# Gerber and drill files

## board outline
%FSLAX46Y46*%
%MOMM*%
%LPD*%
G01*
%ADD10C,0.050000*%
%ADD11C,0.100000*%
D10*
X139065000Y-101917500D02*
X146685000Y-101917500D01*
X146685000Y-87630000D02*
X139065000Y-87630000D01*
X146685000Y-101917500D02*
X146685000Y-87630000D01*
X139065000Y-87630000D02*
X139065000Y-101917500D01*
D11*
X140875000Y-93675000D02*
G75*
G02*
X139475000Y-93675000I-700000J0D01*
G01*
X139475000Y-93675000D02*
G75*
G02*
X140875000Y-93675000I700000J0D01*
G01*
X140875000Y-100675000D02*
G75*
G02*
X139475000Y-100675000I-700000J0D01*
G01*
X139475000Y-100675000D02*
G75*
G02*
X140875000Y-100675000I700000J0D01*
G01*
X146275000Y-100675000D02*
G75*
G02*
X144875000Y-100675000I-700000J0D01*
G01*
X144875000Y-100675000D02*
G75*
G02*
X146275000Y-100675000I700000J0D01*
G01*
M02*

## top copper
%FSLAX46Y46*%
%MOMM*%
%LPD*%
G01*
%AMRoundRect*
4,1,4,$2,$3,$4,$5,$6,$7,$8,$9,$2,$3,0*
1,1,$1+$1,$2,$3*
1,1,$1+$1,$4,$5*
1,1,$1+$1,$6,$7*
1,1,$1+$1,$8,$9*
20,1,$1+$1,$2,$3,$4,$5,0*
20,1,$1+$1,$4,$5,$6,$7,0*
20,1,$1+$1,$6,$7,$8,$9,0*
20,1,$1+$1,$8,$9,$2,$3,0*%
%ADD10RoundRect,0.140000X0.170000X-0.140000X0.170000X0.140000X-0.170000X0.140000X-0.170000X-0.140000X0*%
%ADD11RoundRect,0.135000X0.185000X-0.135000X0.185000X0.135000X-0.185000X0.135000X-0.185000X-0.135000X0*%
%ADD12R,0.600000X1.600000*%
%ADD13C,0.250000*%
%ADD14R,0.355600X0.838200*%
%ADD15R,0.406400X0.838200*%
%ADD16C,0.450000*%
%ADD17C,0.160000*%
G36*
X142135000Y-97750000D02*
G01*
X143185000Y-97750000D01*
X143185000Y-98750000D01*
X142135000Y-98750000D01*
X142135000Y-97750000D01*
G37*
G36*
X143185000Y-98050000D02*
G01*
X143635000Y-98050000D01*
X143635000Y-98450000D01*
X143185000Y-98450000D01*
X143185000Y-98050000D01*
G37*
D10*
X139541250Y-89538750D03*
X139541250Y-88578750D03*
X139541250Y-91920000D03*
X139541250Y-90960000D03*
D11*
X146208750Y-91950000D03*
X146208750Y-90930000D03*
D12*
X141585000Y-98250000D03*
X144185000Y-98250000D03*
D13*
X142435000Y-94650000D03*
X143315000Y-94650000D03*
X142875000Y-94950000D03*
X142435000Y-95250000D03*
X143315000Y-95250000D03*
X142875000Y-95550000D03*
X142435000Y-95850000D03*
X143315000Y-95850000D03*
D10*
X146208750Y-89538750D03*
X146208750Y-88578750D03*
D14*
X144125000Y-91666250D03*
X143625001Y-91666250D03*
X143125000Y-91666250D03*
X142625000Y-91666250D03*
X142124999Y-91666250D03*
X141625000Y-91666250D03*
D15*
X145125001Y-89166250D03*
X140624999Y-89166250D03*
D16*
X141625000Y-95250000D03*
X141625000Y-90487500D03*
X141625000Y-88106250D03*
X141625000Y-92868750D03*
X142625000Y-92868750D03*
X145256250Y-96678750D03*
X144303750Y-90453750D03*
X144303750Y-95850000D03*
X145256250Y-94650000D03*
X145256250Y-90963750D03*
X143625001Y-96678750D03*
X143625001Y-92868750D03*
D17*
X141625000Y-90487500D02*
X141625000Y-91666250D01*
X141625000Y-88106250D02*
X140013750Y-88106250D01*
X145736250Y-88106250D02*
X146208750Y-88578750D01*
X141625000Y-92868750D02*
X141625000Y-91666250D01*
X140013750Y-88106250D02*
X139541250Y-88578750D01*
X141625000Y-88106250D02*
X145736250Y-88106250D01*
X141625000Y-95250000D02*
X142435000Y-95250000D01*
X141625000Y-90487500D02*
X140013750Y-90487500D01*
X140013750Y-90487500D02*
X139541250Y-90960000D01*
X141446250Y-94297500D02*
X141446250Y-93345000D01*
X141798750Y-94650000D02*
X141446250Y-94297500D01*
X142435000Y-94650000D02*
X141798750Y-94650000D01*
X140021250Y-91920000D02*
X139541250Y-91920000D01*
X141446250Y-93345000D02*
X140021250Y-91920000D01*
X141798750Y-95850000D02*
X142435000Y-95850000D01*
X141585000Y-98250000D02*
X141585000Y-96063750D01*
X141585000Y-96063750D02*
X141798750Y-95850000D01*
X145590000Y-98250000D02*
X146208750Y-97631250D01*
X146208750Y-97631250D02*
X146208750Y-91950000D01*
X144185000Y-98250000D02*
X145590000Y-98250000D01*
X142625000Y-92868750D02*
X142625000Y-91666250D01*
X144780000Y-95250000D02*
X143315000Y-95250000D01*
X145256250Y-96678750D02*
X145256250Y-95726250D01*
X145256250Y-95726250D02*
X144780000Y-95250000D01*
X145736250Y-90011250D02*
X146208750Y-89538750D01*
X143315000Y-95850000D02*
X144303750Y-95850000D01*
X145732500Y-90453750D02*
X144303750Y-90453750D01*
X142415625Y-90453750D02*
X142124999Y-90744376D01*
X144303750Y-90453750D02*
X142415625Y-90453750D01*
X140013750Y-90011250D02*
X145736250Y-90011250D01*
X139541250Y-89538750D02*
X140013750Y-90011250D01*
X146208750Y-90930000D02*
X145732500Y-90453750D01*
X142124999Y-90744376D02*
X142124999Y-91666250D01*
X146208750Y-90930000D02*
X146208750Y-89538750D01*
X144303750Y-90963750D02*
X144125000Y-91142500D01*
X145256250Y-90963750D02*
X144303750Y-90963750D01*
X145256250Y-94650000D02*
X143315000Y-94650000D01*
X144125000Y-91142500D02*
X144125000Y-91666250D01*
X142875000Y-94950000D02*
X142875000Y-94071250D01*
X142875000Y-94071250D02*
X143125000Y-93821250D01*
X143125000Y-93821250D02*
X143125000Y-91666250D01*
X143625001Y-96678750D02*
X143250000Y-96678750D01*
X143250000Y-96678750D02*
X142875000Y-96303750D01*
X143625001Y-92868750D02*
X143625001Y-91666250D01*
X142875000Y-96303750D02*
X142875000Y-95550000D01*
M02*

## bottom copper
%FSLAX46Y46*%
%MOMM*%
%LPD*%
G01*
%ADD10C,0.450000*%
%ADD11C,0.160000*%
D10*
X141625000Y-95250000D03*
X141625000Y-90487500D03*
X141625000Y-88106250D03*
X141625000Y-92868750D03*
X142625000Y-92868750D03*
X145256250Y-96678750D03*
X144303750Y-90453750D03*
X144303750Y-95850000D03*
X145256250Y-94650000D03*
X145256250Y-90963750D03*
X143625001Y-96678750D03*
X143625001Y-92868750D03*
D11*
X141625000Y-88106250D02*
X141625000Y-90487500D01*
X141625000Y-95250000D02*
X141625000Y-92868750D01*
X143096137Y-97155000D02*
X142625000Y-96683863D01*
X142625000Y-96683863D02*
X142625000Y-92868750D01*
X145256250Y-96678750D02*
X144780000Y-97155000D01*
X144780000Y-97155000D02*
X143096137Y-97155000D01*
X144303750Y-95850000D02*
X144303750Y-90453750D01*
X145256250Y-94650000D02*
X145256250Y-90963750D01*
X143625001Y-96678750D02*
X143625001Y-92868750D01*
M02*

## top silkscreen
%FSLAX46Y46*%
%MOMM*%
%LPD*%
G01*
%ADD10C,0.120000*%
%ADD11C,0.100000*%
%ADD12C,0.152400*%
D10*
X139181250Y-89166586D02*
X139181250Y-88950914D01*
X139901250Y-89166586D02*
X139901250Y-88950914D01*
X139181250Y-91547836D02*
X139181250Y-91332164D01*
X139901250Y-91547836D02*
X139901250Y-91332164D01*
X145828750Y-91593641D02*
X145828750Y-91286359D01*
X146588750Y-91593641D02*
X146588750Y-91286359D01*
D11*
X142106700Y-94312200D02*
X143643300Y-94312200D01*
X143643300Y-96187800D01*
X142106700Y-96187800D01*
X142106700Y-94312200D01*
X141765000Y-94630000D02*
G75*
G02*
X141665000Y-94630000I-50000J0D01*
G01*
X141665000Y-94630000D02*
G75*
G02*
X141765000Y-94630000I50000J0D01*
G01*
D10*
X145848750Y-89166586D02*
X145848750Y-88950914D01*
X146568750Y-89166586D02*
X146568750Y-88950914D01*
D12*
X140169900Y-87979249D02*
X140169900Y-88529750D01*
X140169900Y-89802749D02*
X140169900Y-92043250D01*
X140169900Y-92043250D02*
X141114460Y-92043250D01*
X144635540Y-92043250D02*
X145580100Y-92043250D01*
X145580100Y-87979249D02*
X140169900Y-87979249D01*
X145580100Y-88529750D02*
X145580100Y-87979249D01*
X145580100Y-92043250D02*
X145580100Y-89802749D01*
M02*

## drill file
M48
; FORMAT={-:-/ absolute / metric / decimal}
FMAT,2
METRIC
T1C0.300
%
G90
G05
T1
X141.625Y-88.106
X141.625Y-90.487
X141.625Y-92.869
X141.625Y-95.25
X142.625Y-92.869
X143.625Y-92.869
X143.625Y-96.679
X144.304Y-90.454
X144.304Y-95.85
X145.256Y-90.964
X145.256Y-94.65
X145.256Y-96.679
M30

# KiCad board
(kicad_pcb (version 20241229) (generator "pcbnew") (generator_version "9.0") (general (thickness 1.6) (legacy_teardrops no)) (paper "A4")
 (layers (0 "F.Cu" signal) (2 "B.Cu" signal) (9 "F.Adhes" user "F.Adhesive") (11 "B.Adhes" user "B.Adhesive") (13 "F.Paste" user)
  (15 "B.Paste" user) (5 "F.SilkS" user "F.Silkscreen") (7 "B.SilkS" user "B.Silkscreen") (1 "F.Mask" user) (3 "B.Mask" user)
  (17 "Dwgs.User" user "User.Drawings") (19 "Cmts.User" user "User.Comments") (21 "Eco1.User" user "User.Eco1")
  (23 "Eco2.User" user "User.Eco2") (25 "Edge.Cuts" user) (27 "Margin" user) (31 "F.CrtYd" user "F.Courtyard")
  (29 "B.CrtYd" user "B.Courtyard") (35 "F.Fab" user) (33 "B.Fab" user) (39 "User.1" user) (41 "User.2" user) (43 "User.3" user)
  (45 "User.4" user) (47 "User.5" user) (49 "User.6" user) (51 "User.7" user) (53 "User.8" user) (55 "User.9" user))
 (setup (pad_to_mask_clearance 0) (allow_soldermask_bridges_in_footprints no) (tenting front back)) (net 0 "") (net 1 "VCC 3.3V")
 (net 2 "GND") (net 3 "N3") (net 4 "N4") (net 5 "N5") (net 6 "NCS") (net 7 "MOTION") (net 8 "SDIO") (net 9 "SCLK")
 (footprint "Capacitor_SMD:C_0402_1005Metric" (layer "F.Cu") (at 139.54125 89.05875 90)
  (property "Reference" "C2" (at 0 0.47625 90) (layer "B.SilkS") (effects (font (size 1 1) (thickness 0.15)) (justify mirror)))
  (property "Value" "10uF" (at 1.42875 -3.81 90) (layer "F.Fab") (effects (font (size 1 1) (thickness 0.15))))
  (fp_line (start -0.107836 -0.36) (end 0.107836 -0.36) (stroke (width 0.12) (type solid)) (layer "F.SilkS"))
  (fp_line (start -0.107836 0.36) (end 0.107836 0.36) (stroke (width 0.12) (type solid)) (layer "F.SilkS"))
  (pad "1" smd roundrect (at -0.48 0 90) (size 0.56 0.62) (layers "F.Cu" "F.Mask" "F.Paste") (roundrect_rratio 0.25) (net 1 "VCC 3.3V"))
  (pad "2" smd roundrect (at 0.48 0 90) (size 0.56 0.62) (layers "F.Cu" "F.Mask" "F.Paste") (roundrect_rratio 0.25) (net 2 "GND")))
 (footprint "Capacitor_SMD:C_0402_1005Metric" (layer "F.Cu") (at 139.54125 91.44 90)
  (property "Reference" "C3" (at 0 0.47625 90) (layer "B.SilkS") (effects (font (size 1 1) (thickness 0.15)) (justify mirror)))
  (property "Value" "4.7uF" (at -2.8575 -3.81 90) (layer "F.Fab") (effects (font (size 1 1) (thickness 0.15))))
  (fp_line (start -0.107836 -0.36) (end 0.107836 -0.36) (stroke (width 0.12) (type solid)) (layer "F.SilkS"))
  (fp_line (start -0.107836 0.36) (end 0.107836 0.36) (stroke (width 0.12) (type solid)) (layer "F.SilkS"))
  (pad "1" smd roundrect (at -0.48 0 90) (size 0.56 0.62) (layers "F.Cu" "F.Mask" "F.Paste") (roundrect_rratio 0.25) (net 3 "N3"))
  (pad "2" smd roundrect (at 0.48 0 90) (size 0.56 0.62) (layers "F.Cu" "F.Mask" "F.Paste") (roundrect_rratio 0.25) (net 2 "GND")))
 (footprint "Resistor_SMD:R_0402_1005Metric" (layer "F.Cu") (at 146.20875 91.44 90)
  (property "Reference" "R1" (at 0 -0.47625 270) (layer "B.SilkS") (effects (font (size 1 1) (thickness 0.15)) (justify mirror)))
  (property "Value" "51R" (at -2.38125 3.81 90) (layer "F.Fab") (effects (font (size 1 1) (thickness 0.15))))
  (fp_line (start -0.153641 -0.38) (end 0.153641 -0.38) (stroke (width 0.12) (type solid)) (layer "F.SilkS"))
  (fp_line (start -0.153641 0.38) (end 0.153641 0.38) (stroke (width 0.12) (type solid)) (layer "F.SilkS"))
  (pad "1" smd roundrect (at -0.51 0 90) (size 0.54 0.64) (layers "F.Cu" "F.Mask" "F.Paste") (roundrect_rratio 0.25) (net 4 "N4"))
  (pad "2" smd roundrect (at 0.51 0 90) (size 0.54 0.64) (layers "F.Cu" "F.Mask" "F.Paste") (roundrect_rratio 0.25) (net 1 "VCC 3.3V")))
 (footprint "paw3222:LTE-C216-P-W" (layer "F.Cu") (at 142.885 98.25 90)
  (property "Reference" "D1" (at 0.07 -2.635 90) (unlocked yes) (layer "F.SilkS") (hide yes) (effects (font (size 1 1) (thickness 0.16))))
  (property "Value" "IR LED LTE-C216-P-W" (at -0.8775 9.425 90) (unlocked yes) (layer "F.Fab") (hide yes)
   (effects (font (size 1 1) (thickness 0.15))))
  (fp_rect (start -0.5 -0.75) (end 0.5 0.3) (stroke (width 0) (type solid)) (fill yes) (layer "F.Cu"))
  (fp_rect (start -0.2 0.3) (end 0.2 0.75) (stroke (width 0) (type solid)) (fill yes) (layer "F.Cu"))
  (pad "1" smd rect (at 0 -1.3 90) (size 1.6 0.6) (layers "F.Cu" "F.Mask" "F.Paste") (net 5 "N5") (thermal_bridge_angle 45))
  (pad "2" smd rect (at 0 1.3 90) (size 1.6 0.6) (layers "F.Cu" "F.Mask" "F.Paste") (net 4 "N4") (thermal_bridge_angle 45)))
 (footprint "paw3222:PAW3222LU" (layer "F.Cu") (at 142.875 95.25)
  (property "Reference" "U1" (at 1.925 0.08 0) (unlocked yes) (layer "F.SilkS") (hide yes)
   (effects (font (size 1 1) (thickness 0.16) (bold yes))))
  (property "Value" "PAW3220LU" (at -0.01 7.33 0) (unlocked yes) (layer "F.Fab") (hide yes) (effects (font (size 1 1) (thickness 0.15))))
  (fp_rect (start -0.7683 -0.9378) (end 0.7683 0.9378) (stroke (width 0.1) (type default)) (fill no) (layer "F.SilkS"))
  (fp_circle (center -1.16 -0.62) (end -1.06 -0.62) (stroke (width 0) (type solid)) (fill yes) (layer "F.SilkS"))
  (fp_circle (center -2.7 -1.575) (end -2 -1.575) (stroke (width 0.1) (type default)) (fill no) (layer "Edge.Cuts"))
  (fp_circle (center -2.7 5.425) (end -2 5.425) (stroke (width 0.1) (type default)) (fill no) (layer "Edge.Cuts"))
  (fp_circle (center 2.7 5.425) (end 3.4 5.425) (stroke (width 0.1) (type default)) (fill no) (layer "Edge.Cuts"))
  (pad "A1" smd circle (at -0.44 -0.6) (size 0.25 0.25) (layers "F.Cu" "F.Mask" "F.Paste") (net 3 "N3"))
  (pad "A3" smd circle (at 0.44 -0.6) (size 0.25 0.25) (layers "F.Cu" "F.Mask" "F.Paste") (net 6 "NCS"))
  (pad "B2" smd circle (at 0 -0.3) (size 0.25 0.25) (layers "F.Cu" "F.Mask" "F.Paste") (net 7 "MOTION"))
  (pad "C1" smd circle (at -0.44 0) (size 0.25 0.25) (layers "F.Cu" "F.Mask" "F.Paste") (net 2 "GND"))
  (pad "C3" smd circle (at 0.44 0) (size 0.25 0.25) (layers "F.Cu" "F.Mask" "F.Paste") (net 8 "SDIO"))
  (pad "D2" smd circle (at 0 0.3) (size 0.25 0.25) (layers "F.Cu" "F.Mask" "F.Paste") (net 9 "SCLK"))
  (pad "E1" smd circle (at -0.44 0.6) (size 0.25 0.25) (layers "F.Cu" "F.Mask" "F.Paste") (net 5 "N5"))
  (pad "E3" smd circle (at 0.44 0.6) (size 0.25 0.25) (layers "F.Cu" "F.Mask" "F.Paste") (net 1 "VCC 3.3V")))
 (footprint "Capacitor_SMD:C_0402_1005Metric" (layer "F.Cu") (at 146.20875 89.05875 90)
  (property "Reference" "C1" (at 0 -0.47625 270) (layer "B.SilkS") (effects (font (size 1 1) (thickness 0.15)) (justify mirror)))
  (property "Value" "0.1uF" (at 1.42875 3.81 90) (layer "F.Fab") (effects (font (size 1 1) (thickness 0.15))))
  (fp_line (start -0.107836 -0.36) (end 0.107836 -0.36) (stroke (width 0.12) (type solid)) (layer "F.SilkS"))
  (fp_line (start -0.107836 0.36) (end 0.107836 0.36) (stroke (width 0.12) (type solid)) (layer "F.SilkS"))
  (pad "1" smd roundrect (at -0.48 0 90) (size 0.56 0.62) (layers "F.Cu" "F.Mask" "F.Paste") (roundrect_rratio 0.25) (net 1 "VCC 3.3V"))
  (pad "2" smd roundrect (at 0.48 0 90) (size 0.56 0.62) (layers "F.Cu" "F.Mask" "F.Paste") (roundrect_rratio 0.25) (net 2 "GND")))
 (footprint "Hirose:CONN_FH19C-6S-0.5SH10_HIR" (layer "F.Cu") (at 142.875 90.01125 180)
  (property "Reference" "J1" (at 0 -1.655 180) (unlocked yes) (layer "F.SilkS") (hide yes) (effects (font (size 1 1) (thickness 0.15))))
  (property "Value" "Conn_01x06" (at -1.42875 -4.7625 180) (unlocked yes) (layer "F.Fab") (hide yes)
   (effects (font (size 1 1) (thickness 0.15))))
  (fp_line (start 2.7051 2.032001) (end 2.7051 1.4815) (stroke (width 0.1524) (type solid)) (layer "F.SilkS"))
  (fp_line (start 2.7051 0.208501) (end 2.7051 -2.032) (stroke (width 0.1524) (type solid)) (layer "F.SilkS"))
  (fp_line (start 2.7051 -2.032) (end 1.76054 -2.032) (stroke (width 0.1524) (type solid)) (layer "F.SilkS"))
  (fp_line (start -1.76054 -2.032) (end -2.7051 -2.032) (stroke (width 0.1524) (type solid)) (layer "F.SilkS"))
  (fp_line (start -2.7051 2.032001) (end 2.7051 2.032001) (stroke (width 0.1524) (type solid)) (layer "F.SilkS"))
  (fp_line (start -2.7051 1.4815) (end -2.7051 2.032001) (stroke (width 0.1524) (type solid)) (layer "F.SilkS"))
  (fp_line (start -2.7051 -2.032) (end -2.7051 0.208501) (stroke (width 0.1524) (type solid)) (layer "F.SilkS"))
  (pad "1" smd rect (at -1.25 -1.655 180) (size 0.3556 0.8382) (layers "F.Cu" "F.Mask" "F.Paste") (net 6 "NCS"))
  (pad "2" smd rect (at -0.750001 -1.655 180) (size 0.3556 0.8382) (layers "F.Cu" "F.Mask" "F.Paste") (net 9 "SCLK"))
  (pad "3" smd rect (at -0.25 -1.655 180) (size 0.3556 0.8382) (layers "F.Cu" "F.Mask" "F.Paste") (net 7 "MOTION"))
  (pad "4" smd rect (at 0.25 -1.655 180) (size 0.3556 0.8382) (layers "F.Cu" "F.Mask" "F.Paste") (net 8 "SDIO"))
  (pad "5" smd rect (at 0.750001 -1.655 180) (size 0.3556 0.8382) (layers "F.Cu" "F.Mask" "F.Paste") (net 1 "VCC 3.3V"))
  (pad "6" smd rect (at 1.25 -1.655 180) (size 0.3556 0.8382) (layers "F.Cu" "F.Mask" "F.Paste") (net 2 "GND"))
  (pad "7" smd rect (at -2.250001 0.845 180) (size 0.4064 0.8382) (layers "F.Cu" "F.Mask" "F.Paste"))
  (pad "8" smd rect (at 2.250001 0.845 180) (size 0.4064 0.8382) (layers "F.Cu" "F.Mask" "F.Paste")))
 (gr_line (start 139.065 101.9175) (end 146.685 101.9175) (stroke (width 0.05) (type default)) (layer "Edge.Cuts"))
 (gr_line (start 146.685 87.63) (end 139.065 87.63) (stroke (width 0.05) (type default)) (layer "Edge.Cuts"))
 (gr_line (start 146.685 101.9175) (end 146.685 87.63) (stroke (width 0.05) (type default)) (layer "Edge.Cuts"))
 (gr_line (start 139.065 87.63) (end 139.065 101.9175) (stroke (width 0.05) (type default)) (layer "Edge.Cuts"))
 (segment (start 141.625 90.4875) (end 141.625 91.66625) (width 0.16) (layer "F.Cu") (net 2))
 (segment (start 141.625 88.10625) (end 140.01375 88.10625) (width 0.16) (layer "F.Cu") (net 2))
 (segment (start 145.73625 88.10625) (end 146.20875 88.57875) (width 0.16) (layer "F.Cu") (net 2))
 (segment (start 141.625 92.86875) (end 141.625 91.66625) (width 0.16) (layer "F.Cu") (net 2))
 (segment (start 140.01375 88.10625) (end 139.54125 88.57875) (width 0.16) (layer "F.Cu") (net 2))
 (segment (start 141.625 88.10625) (end 145.73625 88.10625) (width 0.16) (layer "F.Cu") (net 2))
 (segment (start 141.625 95.25) (end 142.435 95.25) (width 0.16) (layer "F.Cu") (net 2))
 (segment (start 141.625 90.4875) (end 140.01375 90.4875) (width 0.16) (layer "F.Cu") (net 2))
 (segment (start 140.01375 90.4875) (end 139.54125 90.96) (width 0.16) (layer "F.Cu") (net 2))
 (via (at 141.625 95.25) (size 0.45) (drill 0.3) (layers "F.Cu" "B.Cu") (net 2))
 (via (at 141.625 90.4875) (size 0.45) (drill 0.3) (layers "F.Cu" "B.Cu") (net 2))
 (via (at 141.625 88.10625) (size 0.45) (drill 0.3) (layers "F.Cu" "B.Cu") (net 2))
 (via (at 141.625 92.86875) (size 0.45) (drill 0.3) (layers "F.Cu" "B.Cu") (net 2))
 (segment (start 141.625 88.10625) (end 141.625 90.4875) (width 0.16) (layer "B.Cu") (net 2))
 (segment (start 141.625 95.25) (end 141.625 92.86875) (width 0.16) (layer "B.Cu") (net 2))
 (segment (start 141.44625 94.2975) (end 141.44625 93.345) (width 0.16) (layer "F.Cu") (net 3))
 (segment (start 141.79875 94.65) (end 141.44625 94.2975) (width 0.16) (layer "F.Cu") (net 3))
 (segment (start 142.435 94.65) (end 141.79875 94.65) (width 0.16) (layer "F.Cu") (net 3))
 (segment (start 140.02125 91.92) (end 139.54125 91.92) (width 0.16) (layer "F.Cu") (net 3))
 (segment (start 141.44625 93.345) (end 140.02125 91.92) (width 0.16) (layer "F.Cu") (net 3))
 (segment (start 141.79875 95.85) (end 142.435 95.85) (width 0.16) (layer "F.Cu") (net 5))
 (segment (start 141.585 98.25) (end 141.585 96.06375) (width 0.16) (layer "F.Cu") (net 5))
 (segment (start 141.585 96.06375) (end 141.79875 95.85) (width 0.16) (layer "F.Cu") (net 5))
 (segment (start 145.59 98.25) (end 146.20875 97.63125) (width 0.16) (layer "F.Cu") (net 4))
 (segment (start 146.20875 97.63125) (end 146.20875 91.95) (width 0.16) (layer "F.Cu") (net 4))
 (segment (start 144.185 98.25) (end 145.59 98.25) (width 0.16) (layer "F.Cu") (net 4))
 (segment (start 142.625 92.86875) (end 142.625 91.66625) (width 0.16) (layer "F.Cu") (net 8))
 (segment (start 144.78 95.25) (end 143.315 95.25) (width 0.16) (layer "F.Cu") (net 8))
 (segment (start 145.25625 96.67875) (end 145.25625 95.72625) (width 0.16) (layer "F.Cu") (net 8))
 (segment (start 145.25625 95.72625) (end 144.78 95.25) (width 0.16) (layer "F.Cu") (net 8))
 (via (at 142.625 92.86875) (size 0.45) (drill 0.3) (layers "F.Cu" "B.Cu") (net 8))
 (via (at 145.25625 96.67875) (size 0.45) (drill 0.3) (layers "F.Cu" "B.Cu") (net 8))
 (segment (start 143.096137 97.155) (end 142.625 96.683863) (width 0.16) (layer "B.Cu") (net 8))
 (segment (start 142.625 96.683863) (end 142.625 92.86875) (width 0.16) (layer "B.Cu") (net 8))
 (segment (start 145.25625 96.67875) (end 144.78 97.155) (width 0.16) (layer "B.Cu") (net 8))
 (segment (start 144.78 97.155) (end 143.096137 97.155) (width 0.16) (layer "B.Cu") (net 8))
 (segment (start 145.73625 90.01125) (end 146.20875 89.53875) (width 0.16) (layer "F.Cu") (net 1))
 (segment (start 143.315 95.85) (end 144.30375 95.85) (width 0.16) (layer "F.Cu") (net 1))
 (segment (start 145.7325 90.45375) (end 144.30375 90.45375) (width 0.16) (layer "F.Cu") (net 1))
 (segment (start 142.415625 90.45375) (end 142.124999 90.744376) (width 0.16) (layer "F.Cu") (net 1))
 (segment (start 144.30375 90.45375) (end 142.415625 90.45375) (width 0.16) (layer "F.Cu") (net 1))
 (segment (start 140.01375 90.01125) (end 145.73625 90.01125) (width 0.16) (layer "F.Cu") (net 1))
 (segment (start 139.54125 89.53875) (end 140.01375 90.01125) (width 0.16) (layer "F.Cu") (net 1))
 (segment (start 146.20875 90.93) (end 145.7325 90.45375) (width 0.16) (layer "F.Cu") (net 1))
 (segment (start 142.124999 90.744376) (end 142.124999 91.66625) (width 0.16) (layer "F.Cu") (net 1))
 (segment (start 146.20875 90.93) (end 146.20875 89.53875) (width 0.16) (layer "F.Cu") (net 1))
 (via (at 144.30375 90.45375) (size 0.45) (drill 0.3) (layers "F.Cu" "B.Cu") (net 1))
 (via (at 144.30375 95.85) (size 0.45) (drill 0.3) (layers "F.Cu" "B.Cu") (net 1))
 (segment (start 144.30375 95.85) (end 144.30375 90.45375) (width 0.16) (layer "B.Cu") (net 1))
 (segment (start 144.30375 90.96375) (end 144.125 91.1425) (width 0.16) (layer "F.Cu") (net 6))
 (segment (start 145.25625 90.96375) (end 144.30375 90.96375) (width 0.16) (layer "F.Cu") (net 6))
 (segment (start 145.25625 94.65) (end 143.315 94.65) (width 0.16) (layer "F.Cu") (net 6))
 (segment (start 144.125 91.1425) (end 144.125 91.66625) (width 0.16) (layer "F.Cu") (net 6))
 (via (at 145.25625 94.65) (size 0.45) (drill 0.3) (layers "F.Cu" "B.Cu") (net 6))
 (via (at 145.25625 90.96375) (size 0.45) (drill 0.3) (layers "F.Cu" "B.Cu") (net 6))
 (segment (start 145.25625 94.65) (end 145.25625 90.96375) (width 0.16) (layer "B.Cu") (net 6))
 (segment (start 142.875 94.95) (end 142.875 94.07125) (width 0.16) (layer "F.Cu") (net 7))
 (segment (start 142.875 94.07125) (end 143.125 93.82125) (width 0.16) (layer "F.Cu") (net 7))
 (segment (start 143.125 93.82125) (end 143.125 91.66625) (width 0.16) (layer "F.Cu") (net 7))
 (segment (start 143.625001 96.67875) (end 143.25 96.67875) (width 0.16) (layer "F.Cu") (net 9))
 (segment (start 143.25 96.67875) (end 142.875 96.30375) (width 0.16) (layer "F.Cu") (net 9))
 (segment (start 143.625001 92.86875) (end 143.625001 91.66625) (width 0.16) (layer "F.Cu") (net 9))
 (segment (start 142.875 96.30375) (end 142.875 95.55) (width 0.16) (layer "F.Cu") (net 9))
 (via (at 143.625001 96.67875) (size 0.45) (drill 0.3) (layers "F.Cu" "B.Cu") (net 9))
 (via (at 143.625001 92.86875) (size 0.45) (drill 0.3) (layers "F.Cu" "B.Cu") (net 9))
 (segment (start 143.625001 96.67875) (end 143.625001 92.86875) (width 0.16) (layer "B.Cu") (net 9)))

